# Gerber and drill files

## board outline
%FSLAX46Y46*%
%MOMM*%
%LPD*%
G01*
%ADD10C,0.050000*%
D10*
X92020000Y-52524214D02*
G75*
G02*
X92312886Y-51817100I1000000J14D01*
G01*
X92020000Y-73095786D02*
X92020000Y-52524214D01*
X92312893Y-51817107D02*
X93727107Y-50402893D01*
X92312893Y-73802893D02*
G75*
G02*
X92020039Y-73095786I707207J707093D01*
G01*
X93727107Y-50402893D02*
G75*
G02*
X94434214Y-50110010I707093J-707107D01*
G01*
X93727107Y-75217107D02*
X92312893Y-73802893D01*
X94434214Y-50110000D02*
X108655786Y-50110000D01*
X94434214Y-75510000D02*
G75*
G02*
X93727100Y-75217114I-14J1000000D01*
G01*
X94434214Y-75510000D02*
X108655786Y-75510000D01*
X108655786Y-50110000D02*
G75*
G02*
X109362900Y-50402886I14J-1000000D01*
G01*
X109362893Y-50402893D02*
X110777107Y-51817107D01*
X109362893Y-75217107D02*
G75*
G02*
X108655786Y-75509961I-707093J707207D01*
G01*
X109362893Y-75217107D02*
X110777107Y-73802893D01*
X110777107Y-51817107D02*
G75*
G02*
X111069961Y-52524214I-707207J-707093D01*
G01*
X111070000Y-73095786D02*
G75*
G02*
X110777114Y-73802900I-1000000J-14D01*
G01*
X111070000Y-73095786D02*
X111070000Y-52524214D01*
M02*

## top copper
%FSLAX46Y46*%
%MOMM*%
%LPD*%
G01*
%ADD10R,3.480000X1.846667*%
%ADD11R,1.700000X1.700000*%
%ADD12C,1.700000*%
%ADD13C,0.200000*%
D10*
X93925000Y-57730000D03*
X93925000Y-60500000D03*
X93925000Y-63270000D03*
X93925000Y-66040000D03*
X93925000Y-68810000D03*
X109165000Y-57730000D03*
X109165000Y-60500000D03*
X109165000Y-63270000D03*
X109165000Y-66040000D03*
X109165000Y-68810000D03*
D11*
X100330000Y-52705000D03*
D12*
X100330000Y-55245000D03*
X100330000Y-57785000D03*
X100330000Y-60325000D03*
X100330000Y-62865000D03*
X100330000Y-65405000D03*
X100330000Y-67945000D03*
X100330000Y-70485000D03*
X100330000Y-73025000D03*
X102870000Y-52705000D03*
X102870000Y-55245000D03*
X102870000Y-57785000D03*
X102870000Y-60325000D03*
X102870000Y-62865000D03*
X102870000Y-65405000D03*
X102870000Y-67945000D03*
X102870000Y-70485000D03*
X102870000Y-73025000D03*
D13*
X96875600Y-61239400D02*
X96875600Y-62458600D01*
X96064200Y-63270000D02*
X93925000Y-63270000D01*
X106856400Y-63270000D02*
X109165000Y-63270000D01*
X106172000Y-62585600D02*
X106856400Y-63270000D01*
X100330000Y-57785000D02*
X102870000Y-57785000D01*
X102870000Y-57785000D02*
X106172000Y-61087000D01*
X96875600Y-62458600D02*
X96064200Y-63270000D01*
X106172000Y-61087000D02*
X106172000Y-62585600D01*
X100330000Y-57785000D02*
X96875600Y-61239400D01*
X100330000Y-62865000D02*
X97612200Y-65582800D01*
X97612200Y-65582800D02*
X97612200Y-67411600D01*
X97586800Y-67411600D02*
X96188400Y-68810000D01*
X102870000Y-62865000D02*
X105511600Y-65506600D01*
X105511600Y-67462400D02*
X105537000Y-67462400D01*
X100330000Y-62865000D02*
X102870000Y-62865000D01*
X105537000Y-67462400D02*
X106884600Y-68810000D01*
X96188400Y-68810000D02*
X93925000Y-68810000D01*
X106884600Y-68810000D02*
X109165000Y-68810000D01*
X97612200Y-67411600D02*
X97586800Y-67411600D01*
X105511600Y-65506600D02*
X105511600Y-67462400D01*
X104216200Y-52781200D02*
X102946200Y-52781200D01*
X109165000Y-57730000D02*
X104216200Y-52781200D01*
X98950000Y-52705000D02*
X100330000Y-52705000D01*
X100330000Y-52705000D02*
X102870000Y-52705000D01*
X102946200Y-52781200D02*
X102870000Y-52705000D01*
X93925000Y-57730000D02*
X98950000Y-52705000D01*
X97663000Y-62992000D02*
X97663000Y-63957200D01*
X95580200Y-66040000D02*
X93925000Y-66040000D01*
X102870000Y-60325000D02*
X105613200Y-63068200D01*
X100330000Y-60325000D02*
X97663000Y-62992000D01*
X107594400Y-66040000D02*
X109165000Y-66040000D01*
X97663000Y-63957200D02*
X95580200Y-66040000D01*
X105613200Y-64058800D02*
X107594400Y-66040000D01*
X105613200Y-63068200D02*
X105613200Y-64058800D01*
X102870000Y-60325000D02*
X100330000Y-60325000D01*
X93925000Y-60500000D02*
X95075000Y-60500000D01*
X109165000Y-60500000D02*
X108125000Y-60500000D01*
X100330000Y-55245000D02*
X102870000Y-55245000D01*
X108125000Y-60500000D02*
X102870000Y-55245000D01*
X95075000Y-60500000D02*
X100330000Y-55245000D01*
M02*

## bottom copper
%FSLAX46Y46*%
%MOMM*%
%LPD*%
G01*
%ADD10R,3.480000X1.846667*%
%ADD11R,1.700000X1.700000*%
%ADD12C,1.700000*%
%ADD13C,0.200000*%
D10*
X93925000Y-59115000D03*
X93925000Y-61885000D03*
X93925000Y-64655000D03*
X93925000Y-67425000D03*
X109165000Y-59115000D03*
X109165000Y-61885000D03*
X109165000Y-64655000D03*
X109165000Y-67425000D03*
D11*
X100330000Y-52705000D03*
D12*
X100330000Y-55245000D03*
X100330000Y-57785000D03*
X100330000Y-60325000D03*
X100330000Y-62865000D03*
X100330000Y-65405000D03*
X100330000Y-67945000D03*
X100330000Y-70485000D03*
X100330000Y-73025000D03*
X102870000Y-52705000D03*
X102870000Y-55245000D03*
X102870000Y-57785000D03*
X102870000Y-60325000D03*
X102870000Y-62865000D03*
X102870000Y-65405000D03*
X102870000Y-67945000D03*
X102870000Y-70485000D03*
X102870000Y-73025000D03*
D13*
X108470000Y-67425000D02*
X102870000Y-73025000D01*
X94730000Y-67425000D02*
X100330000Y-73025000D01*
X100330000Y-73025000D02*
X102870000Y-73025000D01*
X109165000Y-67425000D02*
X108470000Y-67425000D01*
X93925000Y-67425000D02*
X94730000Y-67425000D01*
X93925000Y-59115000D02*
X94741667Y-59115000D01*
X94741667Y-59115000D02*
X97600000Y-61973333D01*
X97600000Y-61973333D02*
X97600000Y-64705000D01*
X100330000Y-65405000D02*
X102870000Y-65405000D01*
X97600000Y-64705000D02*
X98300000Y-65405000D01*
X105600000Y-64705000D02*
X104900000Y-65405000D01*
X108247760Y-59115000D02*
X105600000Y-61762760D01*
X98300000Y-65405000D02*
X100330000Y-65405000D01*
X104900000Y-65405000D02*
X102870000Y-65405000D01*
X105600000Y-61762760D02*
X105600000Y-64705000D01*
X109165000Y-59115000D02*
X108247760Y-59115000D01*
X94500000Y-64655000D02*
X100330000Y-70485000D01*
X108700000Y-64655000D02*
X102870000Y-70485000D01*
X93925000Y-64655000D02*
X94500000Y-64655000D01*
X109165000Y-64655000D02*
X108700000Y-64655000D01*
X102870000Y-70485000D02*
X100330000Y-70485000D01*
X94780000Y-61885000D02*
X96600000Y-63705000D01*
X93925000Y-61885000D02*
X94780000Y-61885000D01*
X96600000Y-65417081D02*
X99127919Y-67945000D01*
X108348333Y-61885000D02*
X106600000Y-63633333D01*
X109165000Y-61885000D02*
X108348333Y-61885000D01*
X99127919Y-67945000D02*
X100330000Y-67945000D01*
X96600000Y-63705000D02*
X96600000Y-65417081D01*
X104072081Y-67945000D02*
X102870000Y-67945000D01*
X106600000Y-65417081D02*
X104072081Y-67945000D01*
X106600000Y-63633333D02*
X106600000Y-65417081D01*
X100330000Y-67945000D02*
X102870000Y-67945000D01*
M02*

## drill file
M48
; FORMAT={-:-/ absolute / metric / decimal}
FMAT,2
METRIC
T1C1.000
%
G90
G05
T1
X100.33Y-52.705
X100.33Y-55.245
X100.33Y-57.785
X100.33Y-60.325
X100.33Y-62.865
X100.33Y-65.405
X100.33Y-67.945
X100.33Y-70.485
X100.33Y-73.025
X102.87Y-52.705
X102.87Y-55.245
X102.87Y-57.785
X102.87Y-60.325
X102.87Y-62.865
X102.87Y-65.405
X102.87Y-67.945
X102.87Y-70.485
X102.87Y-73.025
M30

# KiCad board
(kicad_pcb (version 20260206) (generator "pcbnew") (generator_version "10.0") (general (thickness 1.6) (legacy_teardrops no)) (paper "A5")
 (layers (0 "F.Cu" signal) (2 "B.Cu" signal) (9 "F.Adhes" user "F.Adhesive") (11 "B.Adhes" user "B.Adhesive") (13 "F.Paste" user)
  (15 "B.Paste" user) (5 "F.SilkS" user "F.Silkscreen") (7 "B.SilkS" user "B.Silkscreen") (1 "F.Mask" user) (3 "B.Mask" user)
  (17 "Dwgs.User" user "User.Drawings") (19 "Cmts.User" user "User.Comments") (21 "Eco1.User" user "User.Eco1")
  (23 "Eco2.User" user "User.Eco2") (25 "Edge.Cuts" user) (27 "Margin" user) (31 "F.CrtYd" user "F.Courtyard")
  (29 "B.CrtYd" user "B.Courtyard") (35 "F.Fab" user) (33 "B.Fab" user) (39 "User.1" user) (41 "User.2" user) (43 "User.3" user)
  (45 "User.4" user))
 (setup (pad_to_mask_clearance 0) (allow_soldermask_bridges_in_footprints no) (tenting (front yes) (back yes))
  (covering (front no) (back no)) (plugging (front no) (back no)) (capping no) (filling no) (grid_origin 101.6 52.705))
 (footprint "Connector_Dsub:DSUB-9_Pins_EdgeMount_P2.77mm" (layer "F.Cu") (at 93.925 63.27 -90)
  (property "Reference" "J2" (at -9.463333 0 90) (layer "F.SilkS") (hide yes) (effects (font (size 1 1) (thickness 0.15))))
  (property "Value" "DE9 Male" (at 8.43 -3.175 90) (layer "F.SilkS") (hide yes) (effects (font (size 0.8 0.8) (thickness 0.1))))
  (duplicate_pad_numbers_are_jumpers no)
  (pad "1" smd rect (at -5.54 0 270) (size 1.846667 3.48) (layers "F.Cu" "F.Mask" "F.Paste") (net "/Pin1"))
  (pad "2" smd rect (at -2.77 0 270) (size 1.846667 3.48) (layers "F.Cu" "F.Mask" "F.Paste") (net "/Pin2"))
  (pad "3" smd rect (at 0 0 270) (size 1.846667 3.48) (layers "F.Cu" "F.Mask" "F.Paste") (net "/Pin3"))
  (pad "4" smd rect (at 2.77 0 270) (size 1.846667 3.48) (layers "F.Cu" "F.Mask" "F.Paste") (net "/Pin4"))
  (pad "5" smd rect (at 5.54 0 270) (size 1.846667 3.48) (layers "F.Cu" "F.Mask" "F.Paste") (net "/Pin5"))
  (pad "6" smd rect (at -4.155 0 270) (size 1.846667 3.48) (layers "B.Cu" "B.Mask" "B.Paste") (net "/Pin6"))
  (pad "7" smd rect (at -1.385 0 270) (size 1.846667 3.48) (layers "B.Cu" "B.Mask" "B.Paste") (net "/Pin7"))
  (pad "8" smd rect (at 1.385 0 270) (size 1.846667 3.48) (layers "B.Cu" "B.Mask" "B.Paste") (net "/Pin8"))
  (pad "9" smd rect (at 4.155 0 270) (size 1.846667 3.48) (layers "B.Cu" "B.Mask" "B.Paste") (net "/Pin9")))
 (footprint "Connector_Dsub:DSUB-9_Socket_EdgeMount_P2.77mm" (layer "F.Cu") (at 109.165 63.27 90)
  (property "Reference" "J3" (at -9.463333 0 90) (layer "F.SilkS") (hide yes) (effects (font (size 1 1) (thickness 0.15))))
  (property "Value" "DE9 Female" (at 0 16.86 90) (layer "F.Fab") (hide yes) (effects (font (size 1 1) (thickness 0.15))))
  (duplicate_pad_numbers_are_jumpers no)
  (pad "1" smd rect (at 5.54 0 90) (size 1.846667 3.48) (layers "F.Cu" "F.Mask" "F.Paste") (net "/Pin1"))
  (pad "2" smd rect (at 2.77 0 90) (size 1.846667 3.48) (layers "F.Cu" "F.Mask" "F.Paste") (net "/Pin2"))
  (pad "3" smd rect (at 0 0 90) (size 1.846667 3.48) (layers "F.Cu" "F.Mask" "F.Paste") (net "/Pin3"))
  (pad "4" smd rect (at -2.77 0 90) (size 1.846667 3.48) (layers "F.Cu" "F.Mask" "F.Paste") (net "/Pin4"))
  (pad "5" smd rect (at -5.54 0 90) (size 1.846667 3.48) (layers "F.Cu" "F.Mask" "F.Paste") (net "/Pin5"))
  (pad "6" smd rect (at 4.155 0 90) (size 1.846667 3.48) (layers "B.Cu" "B.Mask" "B.Paste") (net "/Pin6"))
  (pad "7" smd rect (at 1.385 0 90) (size 1.846667 3.48) (layers "B.Cu" "B.Mask" "B.Paste") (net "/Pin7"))
  (pad "8" smd rect (at -1.385 0 90) (size 1.846667 3.48) (layers "B.Cu" "B.Mask" "B.Paste") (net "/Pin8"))
  (pad "9" smd rect (at -4.155 0 90) (size 1.846667 3.48) (layers "B.Cu" "B.Mask" "B.Paste") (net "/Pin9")))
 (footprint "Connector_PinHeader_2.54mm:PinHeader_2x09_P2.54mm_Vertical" (layer "F.Cu") (at 100.33 52.705)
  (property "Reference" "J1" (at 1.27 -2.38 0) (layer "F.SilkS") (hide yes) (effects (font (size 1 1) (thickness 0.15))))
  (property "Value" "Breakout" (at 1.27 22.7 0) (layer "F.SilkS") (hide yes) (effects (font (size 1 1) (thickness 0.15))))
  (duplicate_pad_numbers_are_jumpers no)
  (pad "a1" thru_hole rect (at 0 0) (size 1.7 1.7) (drill 1) (layers "*.Cu" "*.Mask") (remove_unused_layers no) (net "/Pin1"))
  (pad "a2" thru_hole circle (at 0 2.54) (size 1.7 1.7) (drill 1) (layers "*.Cu" "*.Mask") (remove_unused_layers no) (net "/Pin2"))
  (pad "a3" thru_hole circle (at 0 5.08) (size 1.7 1.7) (drill 1) (layers "*.Cu" "*.Mask") (remove_unused_layers no) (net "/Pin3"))
  (pad "a4" thru_hole circle (at 0 7.62) (size 1.7 1.7) (drill 1) (layers "*.Cu" "*.Mask") (remove_unused_layers no) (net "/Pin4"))
  (pad "a5" thru_hole circle (at 0 10.16) (size 1.7 1.7) (drill 1) (layers "*.Cu" "*.Mask") (remove_unused_layers no) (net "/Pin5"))
  (pad "a6" thru_hole circle (at 0 12.7) (size 1.7 1.7) (drill 1) (layers "*.Cu" "*.Mask") (remove_unused_layers no) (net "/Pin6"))
  (pad "a7" thru_hole circle (at 0 15.24) (size 1.7 1.7) (drill 1) (layers "*.Cu" "*.Mask") (remove_unused_layers no) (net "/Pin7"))
  (pad "a8" thru_hole circle (at 0 17.78) (size 1.7 1.7) (drill 1) (layers "*.Cu" "*.Mask") (remove_unused_layers no) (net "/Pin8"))
  (pad "a9" thru_hole circle (at 0 20.32) (size 1.7 1.7) (drill 1) (layers "*.Cu" "*.Mask") (remove_unused_layers no) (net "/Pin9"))
  (pad "b1" thru_hole circle (at 2.54 0) (size 1.7 1.7) (drill 1) (layers "*.Cu" "*.Mask") (remove_unused_layers no) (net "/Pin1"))
  (pad "b2" thru_hole circle (at 2.54 2.54) (size 1.7 1.7) (drill 1) (layers "*.Cu" "*.Mask") (remove_unused_layers no) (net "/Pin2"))
  (pad "b3" thru_hole circle (at 2.54 5.08) (size 1.7 1.7) (drill 1) (layers "*.Cu" "*.Mask") (remove_unused_layers no) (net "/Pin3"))
  (pad "b4" thru_hole circle (at 2.54 7.62) (size 1.7 1.7) (drill 1) (layers "*.Cu" "*.Mask") (remove_unused_layers no) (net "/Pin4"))
  (pad "b5" thru_hole circle (at 2.54 10.16) (size 1.7 1.7) (drill 1) (layers "*.Cu" "*.Mask") (remove_unused_layers no) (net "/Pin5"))
  (pad "b6" thru_hole circle (at 2.54 12.7) (size 1.7 1.7) (drill 1) (layers "*.Cu" "*.Mask") (remove_unused_layers no) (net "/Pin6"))
  (pad "b7" thru_hole circle (at 2.54 15.24) (size 1.7 1.7) (drill 1) (layers "*.Cu" "*.Mask") (remove_unused_layers no) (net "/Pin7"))
  (pad "b8" thru_hole circle (at 2.54 17.78) (size 1.7 1.7) (drill 1) (layers "*.Cu" "*.Mask") (remove_unused_layers no) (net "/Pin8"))
  (pad "b9" thru_hole circle (at 2.54 20.32) (size 1.7 1.7) (drill 1) (layers "*.Cu" "*.Mask") (remove_unused_layers no) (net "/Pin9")))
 (gr_arc (start 92.02 52.524214) (mid 92.09612 52.141531) (end 92.312893 51.817107) (stroke (width 0.05) (type default)) (layer "Edge.Cuts"))
 (gr_line (start 92.02 73.095786) (end 92.02 52.524214) (stroke (width 0.05) (type default)) (layer "Edge.Cuts"))
 (gr_line (start 92.312893 51.817107) (end 93.727107 50.402893) (stroke (width 0.05) (type default)) (layer "Edge.Cuts"))
 (gr_arc (start 92.312893 73.802893) (mid 92.096125 73.478469) (end 92.02 73.095786) (stroke (width 0.05) (type default))
  (layer "Edge.Cuts"))
 (gr_arc (start 93.727107 50.402893) (mid 94.05153 50.18612) (end 94.434214 50.11) (stroke (width 0.05) (type default)) (layer "Edge.Cuts"))
 (gr_line (start 93.727107 75.217107) (end 92.312893 73.802893) (stroke (width 0.05) (type default)) (layer "Edge.Cuts"))
 (gr_line (start 94.434214 50.11) (end 108.655786 50.11) (stroke (width 0.05) (type default)) (layer "Edge.Cuts"))
 (gr_arc (start 94.434214 75.51) (mid 94.051531 75.43388) (end 93.727107 75.217107) (stroke (width 0.05) (type default)) (layer "Edge.Cuts"))
 (gr_line (start 94.434214 75.51) (end 108.655786 75.51) (stroke (width 0.05) (type default)) (layer "Edge.Cuts"))
 (gr_arc (start 108.655786 50.11) (mid 109.038469 50.18612) (end 109.362893 50.402893) (stroke (width 0.05) (type default))
  (layer "Edge.Cuts"))
 (gr_line (start 109.362893 50.402893) (end 110.777107 51.817107) (stroke (width 0.05) (type default)) (layer "Edge.Cuts"))
 (gr_arc (start 109.362893 75.217107) (mid 109.038469 75.433875) (end 108.655786 75.51) (stroke (width 0.05) (type default))
  (layer "Edge.Cuts"))
 (gr_line (start 109.362893 75.217107) (end 110.777107 73.802893) (stroke (width 0.05) (type default)) (layer "Edge.Cuts"))
 (gr_arc (start 110.777107 51.817107) (mid 110.993875 52.141531) (end 111.07 52.524214) (stroke (width 0.05) (type default))
  (layer "Edge.Cuts"))
 (gr_arc (start 111.07 73.095786) (mid 110.99388 73.478469) (end 110.777107 73.802893) (stroke (width 0.05) (type default))
  (layer "Edge.Cuts"))
 (gr_line (start 111.07 73.095786) (end 111.07 52.524214) (stroke (width 0.05) (type default)) (layer "Edge.Cuts"))
 (segment (start 108.47 67.425) (end 102.87 73.025) (width 0.2) (layer "B.Cu") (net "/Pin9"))
 (segment (start 94.73 67.425) (end 100.33 73.025) (width 0.2) (layer "B.Cu") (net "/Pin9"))
 (segment (start 100.33 73.025) (end 102.87 73.025) (width 0.2) (layer "B.Cu") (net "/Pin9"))
 (segment (start 109.165 67.425) (end 108.47 67.425) (width 0.2) (layer "B.Cu") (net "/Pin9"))
 (segment (start 93.925 67.425) (end 94.73 67.425) (width 0.2) (layer "B.Cu") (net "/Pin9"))
 (segment (start 96.8756 61.2394) (end 96.8756 62.4586) (width 0.2) (layer "F.Cu") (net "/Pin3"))
 (segment (start 96.0642 63.27) (end 93.925 63.27) (width 0.2) (layer "F.Cu") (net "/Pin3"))
 (segment (start 106.8564 63.27) (end 109.165 63.27) (width 0.2) (layer "F.Cu") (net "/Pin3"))
 (segment (start 106.172 62.5856) (end 106.8564 63.27) (width 0.2) (layer "F.Cu") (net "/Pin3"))
 (segment (start 100.33 57.785) (end 102.87 57.785) (width 0.2) (layer "F.Cu") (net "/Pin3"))
 (segment (start 102.87 57.785) (end 106.172 61.087) (width 0.2) (layer "F.Cu") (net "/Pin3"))
 (segment (start 96.8756 62.4586) (end 96.0642 63.27) (width 0.2) (layer "F.Cu") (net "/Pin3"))
 (segment (start 106.172 61.087) (end 106.172 62.5856) (width 0.2) (layer "F.Cu") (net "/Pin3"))
 (segment (start 100.33 57.785) (end 96.8756 61.2394) (width 0.2) (layer "F.Cu") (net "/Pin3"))
 (segment (start 100.33 62.865) (end 97.6122 65.5828) (width 0.2) (layer "F.Cu") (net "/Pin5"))
 (segment (start 97.6122 65.5828) (end 97.6122 67.4116) (width 0.2) (layer "F.Cu") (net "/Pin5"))
 (segment (start 97.5868 67.4116) (end 96.1884 68.81) (width 0.2) (layer "F.Cu") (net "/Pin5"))
 (segment (start 102.87 62.865) (end 105.5116 65.5066) (width 0.2) (layer "F.Cu") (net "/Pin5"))
 (segment (start 105.5116 67.4624) (end 105.537 67.4624) (width 0.2) (layer "F.Cu") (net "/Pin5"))
 (segment (start 100.33 62.865) (end 102.87 62.865) (width 0.2) (layer "F.Cu") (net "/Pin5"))
 (segment (start 105.537 67.4624) (end 106.8846 68.81) (width 0.2) (layer "F.Cu") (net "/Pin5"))
 (segment (start 96.1884 68.81) (end 93.925 68.81) (width 0.2) (layer "F.Cu") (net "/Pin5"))
 (segment (start 106.8846 68.81) (end 109.165 68.81) (width 0.2) (layer "F.Cu") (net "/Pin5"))
 (segment (start 97.6122 67.4116) (end 97.5868 67.4116) (width 0.2) (layer "F.Cu") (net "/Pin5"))
 (segment (start 105.5116 65.5066) (end 105.5116 67.4624) (width 0.2) (layer "F.Cu") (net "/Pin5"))
 (segment (start 104.2162 52.7812) (end 102.9462 52.7812) (width 0.2) (layer "F.Cu") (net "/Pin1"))
 (segment (start 109.165 57.73) (end 104.2162 52.7812) (width 0.2) (layer "F.Cu") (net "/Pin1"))
 (segment (start 98.95 52.705) (end 100.33 52.705) (width 0.2) (layer "F.Cu") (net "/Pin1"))
 (segment (start 100.33 52.705) (end 102.87 52.705) (width 0.2) (layer "F.Cu") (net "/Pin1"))
 (segment (start 102.9462 52.7812) (end 102.87 52.705) (width 0.2) (layer "F.Cu") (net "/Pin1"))
 (segment (start 93.925 57.73) (end 98.95 52.705) (width 0.2) (layer "F.Cu") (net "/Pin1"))
 (segment (start 93.925 59.115) (end 94.741667 59.115) (width 0.2) (layer "B.Cu") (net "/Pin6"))
 (segment (start 94.741667 59.115) (end 97.6 61.973333) (width 0.2) (layer "B.Cu") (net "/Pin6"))
 (segment (start 97.6 61.973333) (end 97.6 64.705) (width 0.2) (layer "B.Cu") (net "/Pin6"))
 (segment (start 100.33 65.405) (end 102.87 65.405) (width 0.2) (layer "B.Cu") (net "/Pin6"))
 (segment (start 97.6 64.705) (end 98.3 65.405) (width 0.2) (layer "B.Cu") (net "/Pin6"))
 (segment (start 105.6 64.705) (end 104.9 65.405) (width 0.2) (layer "B.Cu") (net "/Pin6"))
 (segment (start 108.24776 59.115) (end 105.6 61.76276) (width 0.2) (layer "B.Cu") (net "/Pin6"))
 (segment (start 98.3 65.405) (end 100.33 65.405) (width 0.2) (layer "B.Cu") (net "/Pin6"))
 (segment (start 104.9 65.405) (end 102.87 65.405) (width 0.2) (layer "B.Cu") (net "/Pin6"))
 (segment (start 105.6 61.76276) (end 105.6 64.705) (width 0.2) (layer "B.Cu") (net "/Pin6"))
 (segment (start 109.165 59.115) (end 108.24776 59.115) (width 0.2) (layer "B.Cu") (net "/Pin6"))
 (segment (start 97.663 62.992) (end 97.663 63.9572) (width 0.2) (layer "F.Cu") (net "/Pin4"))
 (segment (start 95.5802 66.04) (end 93.925 66.04) (width 0.2) (layer "F.Cu") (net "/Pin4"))
 (segment (start 102.87 60.325) (end 105.6132 63.0682) (width 0.2) (layer "F.Cu") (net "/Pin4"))
 (segment (start 100.33 60.325) (end 97.663 62.992) (width 0.2) (layer "F.Cu") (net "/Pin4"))
 (segment (start 107.5944 66.04) (end 109.165 66.04) (width 0.2) (layer "F.Cu") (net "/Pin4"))
 (segment (start 97.663 63.9572) (end 95.5802 66.04) (width 0.2) (layer "F.Cu") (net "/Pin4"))
 (segment (start 105.6132 64.0588) (end 107.5944 66.04) (width 0.2) (layer "F.Cu") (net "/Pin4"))
 (segment (start 105.6132 63.0682) (end 105.6132 64.0588) (width 0.2) (layer "F.Cu") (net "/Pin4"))
 (segment (start 102.87 60.325) (end 100.33 60.325) (width 0.2) (layer "F.Cu") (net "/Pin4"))
 (segment (start 94.5 64.655) (end 100.33 70.485) (width 0.2) (layer "B.Cu") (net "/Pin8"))
 (segment (start 108.7 64.655) (end 102.87 70.485) (width 0.2) (layer "B.Cu") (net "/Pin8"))
 (segment (start 93.925 64.655) (end 94.5 64.655) (width 0.2) (layer "B.Cu") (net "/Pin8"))
 (segment (start 109.165 64.655) (end 108.7 64.655) (width 0.2) (layer "B.Cu") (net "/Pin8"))
 (segment (start 102.87 70.485) (end 100.33 70.485) (width 0.2) (layer "B.Cu") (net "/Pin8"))
 (segment (start 93.925 60.5) (end 95.075 60.5) (width 0.2) (layer "F.Cu") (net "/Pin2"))
 (segment (start 109.165 60.5) (end 108.125 60.5) (width 0.2) (layer "F.Cu") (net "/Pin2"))
 (segment (start 100.33 55.245) (end 102.87 55.245) (width 0.2) (layer "F.Cu") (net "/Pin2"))
 (segment (start 108.125 60.5) (end 102.87 55.245) (width 0.2) (layer "F.Cu") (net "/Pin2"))
 (segment (start 95.075 60.5) (end 100.33 55.245) (width 0.2) (layer "F.Cu") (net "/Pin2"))
 (segment (start 94.78 61.885) (end 96.6 63.705) (width 0.2) (layer "B.Cu") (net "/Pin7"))
 (segment (start 93.925 61.885) (end 94.78 61.885) (width 0.2) (layer "B.Cu") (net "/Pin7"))
 (segment (start 96.6 65.417081) (end 99.127919 67.945) (width 0.2) (layer "B.Cu") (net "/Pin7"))
 (segment (start 108.348333 61.885) (end 106.6 63.633333) (width 0.2) (layer "B.Cu") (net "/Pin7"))
 (segment (start 109.165 61.885) (end 108.348333 61.885) (width 0.2) (layer "B.Cu") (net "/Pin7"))
 (segment (start 99.127919 67.945) (end 100.33 67.945) (width 0.2) (layer "B.Cu") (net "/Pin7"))
 (segment (start 96.6 63.705) (end 96.6 65.417081) (width 0.2) (layer "B.Cu") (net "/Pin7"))
 (segment (start 104.072081 67.945) (end 102.87 67.945) (width 0.2) (layer "B.Cu") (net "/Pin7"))
 (segment (start 106.6 65.417081) (end 104.072081 67.945) (width 0.2) (layer "B.Cu") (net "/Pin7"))
 (segment (start 106.6 63.633333) (end 106.6 65.417081) (width 0.2) (layer "B.Cu") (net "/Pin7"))
 (segment (start 100.33 67.945) (end 102.87 67.945) (width 0.2) (layer "B.Cu") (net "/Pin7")))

